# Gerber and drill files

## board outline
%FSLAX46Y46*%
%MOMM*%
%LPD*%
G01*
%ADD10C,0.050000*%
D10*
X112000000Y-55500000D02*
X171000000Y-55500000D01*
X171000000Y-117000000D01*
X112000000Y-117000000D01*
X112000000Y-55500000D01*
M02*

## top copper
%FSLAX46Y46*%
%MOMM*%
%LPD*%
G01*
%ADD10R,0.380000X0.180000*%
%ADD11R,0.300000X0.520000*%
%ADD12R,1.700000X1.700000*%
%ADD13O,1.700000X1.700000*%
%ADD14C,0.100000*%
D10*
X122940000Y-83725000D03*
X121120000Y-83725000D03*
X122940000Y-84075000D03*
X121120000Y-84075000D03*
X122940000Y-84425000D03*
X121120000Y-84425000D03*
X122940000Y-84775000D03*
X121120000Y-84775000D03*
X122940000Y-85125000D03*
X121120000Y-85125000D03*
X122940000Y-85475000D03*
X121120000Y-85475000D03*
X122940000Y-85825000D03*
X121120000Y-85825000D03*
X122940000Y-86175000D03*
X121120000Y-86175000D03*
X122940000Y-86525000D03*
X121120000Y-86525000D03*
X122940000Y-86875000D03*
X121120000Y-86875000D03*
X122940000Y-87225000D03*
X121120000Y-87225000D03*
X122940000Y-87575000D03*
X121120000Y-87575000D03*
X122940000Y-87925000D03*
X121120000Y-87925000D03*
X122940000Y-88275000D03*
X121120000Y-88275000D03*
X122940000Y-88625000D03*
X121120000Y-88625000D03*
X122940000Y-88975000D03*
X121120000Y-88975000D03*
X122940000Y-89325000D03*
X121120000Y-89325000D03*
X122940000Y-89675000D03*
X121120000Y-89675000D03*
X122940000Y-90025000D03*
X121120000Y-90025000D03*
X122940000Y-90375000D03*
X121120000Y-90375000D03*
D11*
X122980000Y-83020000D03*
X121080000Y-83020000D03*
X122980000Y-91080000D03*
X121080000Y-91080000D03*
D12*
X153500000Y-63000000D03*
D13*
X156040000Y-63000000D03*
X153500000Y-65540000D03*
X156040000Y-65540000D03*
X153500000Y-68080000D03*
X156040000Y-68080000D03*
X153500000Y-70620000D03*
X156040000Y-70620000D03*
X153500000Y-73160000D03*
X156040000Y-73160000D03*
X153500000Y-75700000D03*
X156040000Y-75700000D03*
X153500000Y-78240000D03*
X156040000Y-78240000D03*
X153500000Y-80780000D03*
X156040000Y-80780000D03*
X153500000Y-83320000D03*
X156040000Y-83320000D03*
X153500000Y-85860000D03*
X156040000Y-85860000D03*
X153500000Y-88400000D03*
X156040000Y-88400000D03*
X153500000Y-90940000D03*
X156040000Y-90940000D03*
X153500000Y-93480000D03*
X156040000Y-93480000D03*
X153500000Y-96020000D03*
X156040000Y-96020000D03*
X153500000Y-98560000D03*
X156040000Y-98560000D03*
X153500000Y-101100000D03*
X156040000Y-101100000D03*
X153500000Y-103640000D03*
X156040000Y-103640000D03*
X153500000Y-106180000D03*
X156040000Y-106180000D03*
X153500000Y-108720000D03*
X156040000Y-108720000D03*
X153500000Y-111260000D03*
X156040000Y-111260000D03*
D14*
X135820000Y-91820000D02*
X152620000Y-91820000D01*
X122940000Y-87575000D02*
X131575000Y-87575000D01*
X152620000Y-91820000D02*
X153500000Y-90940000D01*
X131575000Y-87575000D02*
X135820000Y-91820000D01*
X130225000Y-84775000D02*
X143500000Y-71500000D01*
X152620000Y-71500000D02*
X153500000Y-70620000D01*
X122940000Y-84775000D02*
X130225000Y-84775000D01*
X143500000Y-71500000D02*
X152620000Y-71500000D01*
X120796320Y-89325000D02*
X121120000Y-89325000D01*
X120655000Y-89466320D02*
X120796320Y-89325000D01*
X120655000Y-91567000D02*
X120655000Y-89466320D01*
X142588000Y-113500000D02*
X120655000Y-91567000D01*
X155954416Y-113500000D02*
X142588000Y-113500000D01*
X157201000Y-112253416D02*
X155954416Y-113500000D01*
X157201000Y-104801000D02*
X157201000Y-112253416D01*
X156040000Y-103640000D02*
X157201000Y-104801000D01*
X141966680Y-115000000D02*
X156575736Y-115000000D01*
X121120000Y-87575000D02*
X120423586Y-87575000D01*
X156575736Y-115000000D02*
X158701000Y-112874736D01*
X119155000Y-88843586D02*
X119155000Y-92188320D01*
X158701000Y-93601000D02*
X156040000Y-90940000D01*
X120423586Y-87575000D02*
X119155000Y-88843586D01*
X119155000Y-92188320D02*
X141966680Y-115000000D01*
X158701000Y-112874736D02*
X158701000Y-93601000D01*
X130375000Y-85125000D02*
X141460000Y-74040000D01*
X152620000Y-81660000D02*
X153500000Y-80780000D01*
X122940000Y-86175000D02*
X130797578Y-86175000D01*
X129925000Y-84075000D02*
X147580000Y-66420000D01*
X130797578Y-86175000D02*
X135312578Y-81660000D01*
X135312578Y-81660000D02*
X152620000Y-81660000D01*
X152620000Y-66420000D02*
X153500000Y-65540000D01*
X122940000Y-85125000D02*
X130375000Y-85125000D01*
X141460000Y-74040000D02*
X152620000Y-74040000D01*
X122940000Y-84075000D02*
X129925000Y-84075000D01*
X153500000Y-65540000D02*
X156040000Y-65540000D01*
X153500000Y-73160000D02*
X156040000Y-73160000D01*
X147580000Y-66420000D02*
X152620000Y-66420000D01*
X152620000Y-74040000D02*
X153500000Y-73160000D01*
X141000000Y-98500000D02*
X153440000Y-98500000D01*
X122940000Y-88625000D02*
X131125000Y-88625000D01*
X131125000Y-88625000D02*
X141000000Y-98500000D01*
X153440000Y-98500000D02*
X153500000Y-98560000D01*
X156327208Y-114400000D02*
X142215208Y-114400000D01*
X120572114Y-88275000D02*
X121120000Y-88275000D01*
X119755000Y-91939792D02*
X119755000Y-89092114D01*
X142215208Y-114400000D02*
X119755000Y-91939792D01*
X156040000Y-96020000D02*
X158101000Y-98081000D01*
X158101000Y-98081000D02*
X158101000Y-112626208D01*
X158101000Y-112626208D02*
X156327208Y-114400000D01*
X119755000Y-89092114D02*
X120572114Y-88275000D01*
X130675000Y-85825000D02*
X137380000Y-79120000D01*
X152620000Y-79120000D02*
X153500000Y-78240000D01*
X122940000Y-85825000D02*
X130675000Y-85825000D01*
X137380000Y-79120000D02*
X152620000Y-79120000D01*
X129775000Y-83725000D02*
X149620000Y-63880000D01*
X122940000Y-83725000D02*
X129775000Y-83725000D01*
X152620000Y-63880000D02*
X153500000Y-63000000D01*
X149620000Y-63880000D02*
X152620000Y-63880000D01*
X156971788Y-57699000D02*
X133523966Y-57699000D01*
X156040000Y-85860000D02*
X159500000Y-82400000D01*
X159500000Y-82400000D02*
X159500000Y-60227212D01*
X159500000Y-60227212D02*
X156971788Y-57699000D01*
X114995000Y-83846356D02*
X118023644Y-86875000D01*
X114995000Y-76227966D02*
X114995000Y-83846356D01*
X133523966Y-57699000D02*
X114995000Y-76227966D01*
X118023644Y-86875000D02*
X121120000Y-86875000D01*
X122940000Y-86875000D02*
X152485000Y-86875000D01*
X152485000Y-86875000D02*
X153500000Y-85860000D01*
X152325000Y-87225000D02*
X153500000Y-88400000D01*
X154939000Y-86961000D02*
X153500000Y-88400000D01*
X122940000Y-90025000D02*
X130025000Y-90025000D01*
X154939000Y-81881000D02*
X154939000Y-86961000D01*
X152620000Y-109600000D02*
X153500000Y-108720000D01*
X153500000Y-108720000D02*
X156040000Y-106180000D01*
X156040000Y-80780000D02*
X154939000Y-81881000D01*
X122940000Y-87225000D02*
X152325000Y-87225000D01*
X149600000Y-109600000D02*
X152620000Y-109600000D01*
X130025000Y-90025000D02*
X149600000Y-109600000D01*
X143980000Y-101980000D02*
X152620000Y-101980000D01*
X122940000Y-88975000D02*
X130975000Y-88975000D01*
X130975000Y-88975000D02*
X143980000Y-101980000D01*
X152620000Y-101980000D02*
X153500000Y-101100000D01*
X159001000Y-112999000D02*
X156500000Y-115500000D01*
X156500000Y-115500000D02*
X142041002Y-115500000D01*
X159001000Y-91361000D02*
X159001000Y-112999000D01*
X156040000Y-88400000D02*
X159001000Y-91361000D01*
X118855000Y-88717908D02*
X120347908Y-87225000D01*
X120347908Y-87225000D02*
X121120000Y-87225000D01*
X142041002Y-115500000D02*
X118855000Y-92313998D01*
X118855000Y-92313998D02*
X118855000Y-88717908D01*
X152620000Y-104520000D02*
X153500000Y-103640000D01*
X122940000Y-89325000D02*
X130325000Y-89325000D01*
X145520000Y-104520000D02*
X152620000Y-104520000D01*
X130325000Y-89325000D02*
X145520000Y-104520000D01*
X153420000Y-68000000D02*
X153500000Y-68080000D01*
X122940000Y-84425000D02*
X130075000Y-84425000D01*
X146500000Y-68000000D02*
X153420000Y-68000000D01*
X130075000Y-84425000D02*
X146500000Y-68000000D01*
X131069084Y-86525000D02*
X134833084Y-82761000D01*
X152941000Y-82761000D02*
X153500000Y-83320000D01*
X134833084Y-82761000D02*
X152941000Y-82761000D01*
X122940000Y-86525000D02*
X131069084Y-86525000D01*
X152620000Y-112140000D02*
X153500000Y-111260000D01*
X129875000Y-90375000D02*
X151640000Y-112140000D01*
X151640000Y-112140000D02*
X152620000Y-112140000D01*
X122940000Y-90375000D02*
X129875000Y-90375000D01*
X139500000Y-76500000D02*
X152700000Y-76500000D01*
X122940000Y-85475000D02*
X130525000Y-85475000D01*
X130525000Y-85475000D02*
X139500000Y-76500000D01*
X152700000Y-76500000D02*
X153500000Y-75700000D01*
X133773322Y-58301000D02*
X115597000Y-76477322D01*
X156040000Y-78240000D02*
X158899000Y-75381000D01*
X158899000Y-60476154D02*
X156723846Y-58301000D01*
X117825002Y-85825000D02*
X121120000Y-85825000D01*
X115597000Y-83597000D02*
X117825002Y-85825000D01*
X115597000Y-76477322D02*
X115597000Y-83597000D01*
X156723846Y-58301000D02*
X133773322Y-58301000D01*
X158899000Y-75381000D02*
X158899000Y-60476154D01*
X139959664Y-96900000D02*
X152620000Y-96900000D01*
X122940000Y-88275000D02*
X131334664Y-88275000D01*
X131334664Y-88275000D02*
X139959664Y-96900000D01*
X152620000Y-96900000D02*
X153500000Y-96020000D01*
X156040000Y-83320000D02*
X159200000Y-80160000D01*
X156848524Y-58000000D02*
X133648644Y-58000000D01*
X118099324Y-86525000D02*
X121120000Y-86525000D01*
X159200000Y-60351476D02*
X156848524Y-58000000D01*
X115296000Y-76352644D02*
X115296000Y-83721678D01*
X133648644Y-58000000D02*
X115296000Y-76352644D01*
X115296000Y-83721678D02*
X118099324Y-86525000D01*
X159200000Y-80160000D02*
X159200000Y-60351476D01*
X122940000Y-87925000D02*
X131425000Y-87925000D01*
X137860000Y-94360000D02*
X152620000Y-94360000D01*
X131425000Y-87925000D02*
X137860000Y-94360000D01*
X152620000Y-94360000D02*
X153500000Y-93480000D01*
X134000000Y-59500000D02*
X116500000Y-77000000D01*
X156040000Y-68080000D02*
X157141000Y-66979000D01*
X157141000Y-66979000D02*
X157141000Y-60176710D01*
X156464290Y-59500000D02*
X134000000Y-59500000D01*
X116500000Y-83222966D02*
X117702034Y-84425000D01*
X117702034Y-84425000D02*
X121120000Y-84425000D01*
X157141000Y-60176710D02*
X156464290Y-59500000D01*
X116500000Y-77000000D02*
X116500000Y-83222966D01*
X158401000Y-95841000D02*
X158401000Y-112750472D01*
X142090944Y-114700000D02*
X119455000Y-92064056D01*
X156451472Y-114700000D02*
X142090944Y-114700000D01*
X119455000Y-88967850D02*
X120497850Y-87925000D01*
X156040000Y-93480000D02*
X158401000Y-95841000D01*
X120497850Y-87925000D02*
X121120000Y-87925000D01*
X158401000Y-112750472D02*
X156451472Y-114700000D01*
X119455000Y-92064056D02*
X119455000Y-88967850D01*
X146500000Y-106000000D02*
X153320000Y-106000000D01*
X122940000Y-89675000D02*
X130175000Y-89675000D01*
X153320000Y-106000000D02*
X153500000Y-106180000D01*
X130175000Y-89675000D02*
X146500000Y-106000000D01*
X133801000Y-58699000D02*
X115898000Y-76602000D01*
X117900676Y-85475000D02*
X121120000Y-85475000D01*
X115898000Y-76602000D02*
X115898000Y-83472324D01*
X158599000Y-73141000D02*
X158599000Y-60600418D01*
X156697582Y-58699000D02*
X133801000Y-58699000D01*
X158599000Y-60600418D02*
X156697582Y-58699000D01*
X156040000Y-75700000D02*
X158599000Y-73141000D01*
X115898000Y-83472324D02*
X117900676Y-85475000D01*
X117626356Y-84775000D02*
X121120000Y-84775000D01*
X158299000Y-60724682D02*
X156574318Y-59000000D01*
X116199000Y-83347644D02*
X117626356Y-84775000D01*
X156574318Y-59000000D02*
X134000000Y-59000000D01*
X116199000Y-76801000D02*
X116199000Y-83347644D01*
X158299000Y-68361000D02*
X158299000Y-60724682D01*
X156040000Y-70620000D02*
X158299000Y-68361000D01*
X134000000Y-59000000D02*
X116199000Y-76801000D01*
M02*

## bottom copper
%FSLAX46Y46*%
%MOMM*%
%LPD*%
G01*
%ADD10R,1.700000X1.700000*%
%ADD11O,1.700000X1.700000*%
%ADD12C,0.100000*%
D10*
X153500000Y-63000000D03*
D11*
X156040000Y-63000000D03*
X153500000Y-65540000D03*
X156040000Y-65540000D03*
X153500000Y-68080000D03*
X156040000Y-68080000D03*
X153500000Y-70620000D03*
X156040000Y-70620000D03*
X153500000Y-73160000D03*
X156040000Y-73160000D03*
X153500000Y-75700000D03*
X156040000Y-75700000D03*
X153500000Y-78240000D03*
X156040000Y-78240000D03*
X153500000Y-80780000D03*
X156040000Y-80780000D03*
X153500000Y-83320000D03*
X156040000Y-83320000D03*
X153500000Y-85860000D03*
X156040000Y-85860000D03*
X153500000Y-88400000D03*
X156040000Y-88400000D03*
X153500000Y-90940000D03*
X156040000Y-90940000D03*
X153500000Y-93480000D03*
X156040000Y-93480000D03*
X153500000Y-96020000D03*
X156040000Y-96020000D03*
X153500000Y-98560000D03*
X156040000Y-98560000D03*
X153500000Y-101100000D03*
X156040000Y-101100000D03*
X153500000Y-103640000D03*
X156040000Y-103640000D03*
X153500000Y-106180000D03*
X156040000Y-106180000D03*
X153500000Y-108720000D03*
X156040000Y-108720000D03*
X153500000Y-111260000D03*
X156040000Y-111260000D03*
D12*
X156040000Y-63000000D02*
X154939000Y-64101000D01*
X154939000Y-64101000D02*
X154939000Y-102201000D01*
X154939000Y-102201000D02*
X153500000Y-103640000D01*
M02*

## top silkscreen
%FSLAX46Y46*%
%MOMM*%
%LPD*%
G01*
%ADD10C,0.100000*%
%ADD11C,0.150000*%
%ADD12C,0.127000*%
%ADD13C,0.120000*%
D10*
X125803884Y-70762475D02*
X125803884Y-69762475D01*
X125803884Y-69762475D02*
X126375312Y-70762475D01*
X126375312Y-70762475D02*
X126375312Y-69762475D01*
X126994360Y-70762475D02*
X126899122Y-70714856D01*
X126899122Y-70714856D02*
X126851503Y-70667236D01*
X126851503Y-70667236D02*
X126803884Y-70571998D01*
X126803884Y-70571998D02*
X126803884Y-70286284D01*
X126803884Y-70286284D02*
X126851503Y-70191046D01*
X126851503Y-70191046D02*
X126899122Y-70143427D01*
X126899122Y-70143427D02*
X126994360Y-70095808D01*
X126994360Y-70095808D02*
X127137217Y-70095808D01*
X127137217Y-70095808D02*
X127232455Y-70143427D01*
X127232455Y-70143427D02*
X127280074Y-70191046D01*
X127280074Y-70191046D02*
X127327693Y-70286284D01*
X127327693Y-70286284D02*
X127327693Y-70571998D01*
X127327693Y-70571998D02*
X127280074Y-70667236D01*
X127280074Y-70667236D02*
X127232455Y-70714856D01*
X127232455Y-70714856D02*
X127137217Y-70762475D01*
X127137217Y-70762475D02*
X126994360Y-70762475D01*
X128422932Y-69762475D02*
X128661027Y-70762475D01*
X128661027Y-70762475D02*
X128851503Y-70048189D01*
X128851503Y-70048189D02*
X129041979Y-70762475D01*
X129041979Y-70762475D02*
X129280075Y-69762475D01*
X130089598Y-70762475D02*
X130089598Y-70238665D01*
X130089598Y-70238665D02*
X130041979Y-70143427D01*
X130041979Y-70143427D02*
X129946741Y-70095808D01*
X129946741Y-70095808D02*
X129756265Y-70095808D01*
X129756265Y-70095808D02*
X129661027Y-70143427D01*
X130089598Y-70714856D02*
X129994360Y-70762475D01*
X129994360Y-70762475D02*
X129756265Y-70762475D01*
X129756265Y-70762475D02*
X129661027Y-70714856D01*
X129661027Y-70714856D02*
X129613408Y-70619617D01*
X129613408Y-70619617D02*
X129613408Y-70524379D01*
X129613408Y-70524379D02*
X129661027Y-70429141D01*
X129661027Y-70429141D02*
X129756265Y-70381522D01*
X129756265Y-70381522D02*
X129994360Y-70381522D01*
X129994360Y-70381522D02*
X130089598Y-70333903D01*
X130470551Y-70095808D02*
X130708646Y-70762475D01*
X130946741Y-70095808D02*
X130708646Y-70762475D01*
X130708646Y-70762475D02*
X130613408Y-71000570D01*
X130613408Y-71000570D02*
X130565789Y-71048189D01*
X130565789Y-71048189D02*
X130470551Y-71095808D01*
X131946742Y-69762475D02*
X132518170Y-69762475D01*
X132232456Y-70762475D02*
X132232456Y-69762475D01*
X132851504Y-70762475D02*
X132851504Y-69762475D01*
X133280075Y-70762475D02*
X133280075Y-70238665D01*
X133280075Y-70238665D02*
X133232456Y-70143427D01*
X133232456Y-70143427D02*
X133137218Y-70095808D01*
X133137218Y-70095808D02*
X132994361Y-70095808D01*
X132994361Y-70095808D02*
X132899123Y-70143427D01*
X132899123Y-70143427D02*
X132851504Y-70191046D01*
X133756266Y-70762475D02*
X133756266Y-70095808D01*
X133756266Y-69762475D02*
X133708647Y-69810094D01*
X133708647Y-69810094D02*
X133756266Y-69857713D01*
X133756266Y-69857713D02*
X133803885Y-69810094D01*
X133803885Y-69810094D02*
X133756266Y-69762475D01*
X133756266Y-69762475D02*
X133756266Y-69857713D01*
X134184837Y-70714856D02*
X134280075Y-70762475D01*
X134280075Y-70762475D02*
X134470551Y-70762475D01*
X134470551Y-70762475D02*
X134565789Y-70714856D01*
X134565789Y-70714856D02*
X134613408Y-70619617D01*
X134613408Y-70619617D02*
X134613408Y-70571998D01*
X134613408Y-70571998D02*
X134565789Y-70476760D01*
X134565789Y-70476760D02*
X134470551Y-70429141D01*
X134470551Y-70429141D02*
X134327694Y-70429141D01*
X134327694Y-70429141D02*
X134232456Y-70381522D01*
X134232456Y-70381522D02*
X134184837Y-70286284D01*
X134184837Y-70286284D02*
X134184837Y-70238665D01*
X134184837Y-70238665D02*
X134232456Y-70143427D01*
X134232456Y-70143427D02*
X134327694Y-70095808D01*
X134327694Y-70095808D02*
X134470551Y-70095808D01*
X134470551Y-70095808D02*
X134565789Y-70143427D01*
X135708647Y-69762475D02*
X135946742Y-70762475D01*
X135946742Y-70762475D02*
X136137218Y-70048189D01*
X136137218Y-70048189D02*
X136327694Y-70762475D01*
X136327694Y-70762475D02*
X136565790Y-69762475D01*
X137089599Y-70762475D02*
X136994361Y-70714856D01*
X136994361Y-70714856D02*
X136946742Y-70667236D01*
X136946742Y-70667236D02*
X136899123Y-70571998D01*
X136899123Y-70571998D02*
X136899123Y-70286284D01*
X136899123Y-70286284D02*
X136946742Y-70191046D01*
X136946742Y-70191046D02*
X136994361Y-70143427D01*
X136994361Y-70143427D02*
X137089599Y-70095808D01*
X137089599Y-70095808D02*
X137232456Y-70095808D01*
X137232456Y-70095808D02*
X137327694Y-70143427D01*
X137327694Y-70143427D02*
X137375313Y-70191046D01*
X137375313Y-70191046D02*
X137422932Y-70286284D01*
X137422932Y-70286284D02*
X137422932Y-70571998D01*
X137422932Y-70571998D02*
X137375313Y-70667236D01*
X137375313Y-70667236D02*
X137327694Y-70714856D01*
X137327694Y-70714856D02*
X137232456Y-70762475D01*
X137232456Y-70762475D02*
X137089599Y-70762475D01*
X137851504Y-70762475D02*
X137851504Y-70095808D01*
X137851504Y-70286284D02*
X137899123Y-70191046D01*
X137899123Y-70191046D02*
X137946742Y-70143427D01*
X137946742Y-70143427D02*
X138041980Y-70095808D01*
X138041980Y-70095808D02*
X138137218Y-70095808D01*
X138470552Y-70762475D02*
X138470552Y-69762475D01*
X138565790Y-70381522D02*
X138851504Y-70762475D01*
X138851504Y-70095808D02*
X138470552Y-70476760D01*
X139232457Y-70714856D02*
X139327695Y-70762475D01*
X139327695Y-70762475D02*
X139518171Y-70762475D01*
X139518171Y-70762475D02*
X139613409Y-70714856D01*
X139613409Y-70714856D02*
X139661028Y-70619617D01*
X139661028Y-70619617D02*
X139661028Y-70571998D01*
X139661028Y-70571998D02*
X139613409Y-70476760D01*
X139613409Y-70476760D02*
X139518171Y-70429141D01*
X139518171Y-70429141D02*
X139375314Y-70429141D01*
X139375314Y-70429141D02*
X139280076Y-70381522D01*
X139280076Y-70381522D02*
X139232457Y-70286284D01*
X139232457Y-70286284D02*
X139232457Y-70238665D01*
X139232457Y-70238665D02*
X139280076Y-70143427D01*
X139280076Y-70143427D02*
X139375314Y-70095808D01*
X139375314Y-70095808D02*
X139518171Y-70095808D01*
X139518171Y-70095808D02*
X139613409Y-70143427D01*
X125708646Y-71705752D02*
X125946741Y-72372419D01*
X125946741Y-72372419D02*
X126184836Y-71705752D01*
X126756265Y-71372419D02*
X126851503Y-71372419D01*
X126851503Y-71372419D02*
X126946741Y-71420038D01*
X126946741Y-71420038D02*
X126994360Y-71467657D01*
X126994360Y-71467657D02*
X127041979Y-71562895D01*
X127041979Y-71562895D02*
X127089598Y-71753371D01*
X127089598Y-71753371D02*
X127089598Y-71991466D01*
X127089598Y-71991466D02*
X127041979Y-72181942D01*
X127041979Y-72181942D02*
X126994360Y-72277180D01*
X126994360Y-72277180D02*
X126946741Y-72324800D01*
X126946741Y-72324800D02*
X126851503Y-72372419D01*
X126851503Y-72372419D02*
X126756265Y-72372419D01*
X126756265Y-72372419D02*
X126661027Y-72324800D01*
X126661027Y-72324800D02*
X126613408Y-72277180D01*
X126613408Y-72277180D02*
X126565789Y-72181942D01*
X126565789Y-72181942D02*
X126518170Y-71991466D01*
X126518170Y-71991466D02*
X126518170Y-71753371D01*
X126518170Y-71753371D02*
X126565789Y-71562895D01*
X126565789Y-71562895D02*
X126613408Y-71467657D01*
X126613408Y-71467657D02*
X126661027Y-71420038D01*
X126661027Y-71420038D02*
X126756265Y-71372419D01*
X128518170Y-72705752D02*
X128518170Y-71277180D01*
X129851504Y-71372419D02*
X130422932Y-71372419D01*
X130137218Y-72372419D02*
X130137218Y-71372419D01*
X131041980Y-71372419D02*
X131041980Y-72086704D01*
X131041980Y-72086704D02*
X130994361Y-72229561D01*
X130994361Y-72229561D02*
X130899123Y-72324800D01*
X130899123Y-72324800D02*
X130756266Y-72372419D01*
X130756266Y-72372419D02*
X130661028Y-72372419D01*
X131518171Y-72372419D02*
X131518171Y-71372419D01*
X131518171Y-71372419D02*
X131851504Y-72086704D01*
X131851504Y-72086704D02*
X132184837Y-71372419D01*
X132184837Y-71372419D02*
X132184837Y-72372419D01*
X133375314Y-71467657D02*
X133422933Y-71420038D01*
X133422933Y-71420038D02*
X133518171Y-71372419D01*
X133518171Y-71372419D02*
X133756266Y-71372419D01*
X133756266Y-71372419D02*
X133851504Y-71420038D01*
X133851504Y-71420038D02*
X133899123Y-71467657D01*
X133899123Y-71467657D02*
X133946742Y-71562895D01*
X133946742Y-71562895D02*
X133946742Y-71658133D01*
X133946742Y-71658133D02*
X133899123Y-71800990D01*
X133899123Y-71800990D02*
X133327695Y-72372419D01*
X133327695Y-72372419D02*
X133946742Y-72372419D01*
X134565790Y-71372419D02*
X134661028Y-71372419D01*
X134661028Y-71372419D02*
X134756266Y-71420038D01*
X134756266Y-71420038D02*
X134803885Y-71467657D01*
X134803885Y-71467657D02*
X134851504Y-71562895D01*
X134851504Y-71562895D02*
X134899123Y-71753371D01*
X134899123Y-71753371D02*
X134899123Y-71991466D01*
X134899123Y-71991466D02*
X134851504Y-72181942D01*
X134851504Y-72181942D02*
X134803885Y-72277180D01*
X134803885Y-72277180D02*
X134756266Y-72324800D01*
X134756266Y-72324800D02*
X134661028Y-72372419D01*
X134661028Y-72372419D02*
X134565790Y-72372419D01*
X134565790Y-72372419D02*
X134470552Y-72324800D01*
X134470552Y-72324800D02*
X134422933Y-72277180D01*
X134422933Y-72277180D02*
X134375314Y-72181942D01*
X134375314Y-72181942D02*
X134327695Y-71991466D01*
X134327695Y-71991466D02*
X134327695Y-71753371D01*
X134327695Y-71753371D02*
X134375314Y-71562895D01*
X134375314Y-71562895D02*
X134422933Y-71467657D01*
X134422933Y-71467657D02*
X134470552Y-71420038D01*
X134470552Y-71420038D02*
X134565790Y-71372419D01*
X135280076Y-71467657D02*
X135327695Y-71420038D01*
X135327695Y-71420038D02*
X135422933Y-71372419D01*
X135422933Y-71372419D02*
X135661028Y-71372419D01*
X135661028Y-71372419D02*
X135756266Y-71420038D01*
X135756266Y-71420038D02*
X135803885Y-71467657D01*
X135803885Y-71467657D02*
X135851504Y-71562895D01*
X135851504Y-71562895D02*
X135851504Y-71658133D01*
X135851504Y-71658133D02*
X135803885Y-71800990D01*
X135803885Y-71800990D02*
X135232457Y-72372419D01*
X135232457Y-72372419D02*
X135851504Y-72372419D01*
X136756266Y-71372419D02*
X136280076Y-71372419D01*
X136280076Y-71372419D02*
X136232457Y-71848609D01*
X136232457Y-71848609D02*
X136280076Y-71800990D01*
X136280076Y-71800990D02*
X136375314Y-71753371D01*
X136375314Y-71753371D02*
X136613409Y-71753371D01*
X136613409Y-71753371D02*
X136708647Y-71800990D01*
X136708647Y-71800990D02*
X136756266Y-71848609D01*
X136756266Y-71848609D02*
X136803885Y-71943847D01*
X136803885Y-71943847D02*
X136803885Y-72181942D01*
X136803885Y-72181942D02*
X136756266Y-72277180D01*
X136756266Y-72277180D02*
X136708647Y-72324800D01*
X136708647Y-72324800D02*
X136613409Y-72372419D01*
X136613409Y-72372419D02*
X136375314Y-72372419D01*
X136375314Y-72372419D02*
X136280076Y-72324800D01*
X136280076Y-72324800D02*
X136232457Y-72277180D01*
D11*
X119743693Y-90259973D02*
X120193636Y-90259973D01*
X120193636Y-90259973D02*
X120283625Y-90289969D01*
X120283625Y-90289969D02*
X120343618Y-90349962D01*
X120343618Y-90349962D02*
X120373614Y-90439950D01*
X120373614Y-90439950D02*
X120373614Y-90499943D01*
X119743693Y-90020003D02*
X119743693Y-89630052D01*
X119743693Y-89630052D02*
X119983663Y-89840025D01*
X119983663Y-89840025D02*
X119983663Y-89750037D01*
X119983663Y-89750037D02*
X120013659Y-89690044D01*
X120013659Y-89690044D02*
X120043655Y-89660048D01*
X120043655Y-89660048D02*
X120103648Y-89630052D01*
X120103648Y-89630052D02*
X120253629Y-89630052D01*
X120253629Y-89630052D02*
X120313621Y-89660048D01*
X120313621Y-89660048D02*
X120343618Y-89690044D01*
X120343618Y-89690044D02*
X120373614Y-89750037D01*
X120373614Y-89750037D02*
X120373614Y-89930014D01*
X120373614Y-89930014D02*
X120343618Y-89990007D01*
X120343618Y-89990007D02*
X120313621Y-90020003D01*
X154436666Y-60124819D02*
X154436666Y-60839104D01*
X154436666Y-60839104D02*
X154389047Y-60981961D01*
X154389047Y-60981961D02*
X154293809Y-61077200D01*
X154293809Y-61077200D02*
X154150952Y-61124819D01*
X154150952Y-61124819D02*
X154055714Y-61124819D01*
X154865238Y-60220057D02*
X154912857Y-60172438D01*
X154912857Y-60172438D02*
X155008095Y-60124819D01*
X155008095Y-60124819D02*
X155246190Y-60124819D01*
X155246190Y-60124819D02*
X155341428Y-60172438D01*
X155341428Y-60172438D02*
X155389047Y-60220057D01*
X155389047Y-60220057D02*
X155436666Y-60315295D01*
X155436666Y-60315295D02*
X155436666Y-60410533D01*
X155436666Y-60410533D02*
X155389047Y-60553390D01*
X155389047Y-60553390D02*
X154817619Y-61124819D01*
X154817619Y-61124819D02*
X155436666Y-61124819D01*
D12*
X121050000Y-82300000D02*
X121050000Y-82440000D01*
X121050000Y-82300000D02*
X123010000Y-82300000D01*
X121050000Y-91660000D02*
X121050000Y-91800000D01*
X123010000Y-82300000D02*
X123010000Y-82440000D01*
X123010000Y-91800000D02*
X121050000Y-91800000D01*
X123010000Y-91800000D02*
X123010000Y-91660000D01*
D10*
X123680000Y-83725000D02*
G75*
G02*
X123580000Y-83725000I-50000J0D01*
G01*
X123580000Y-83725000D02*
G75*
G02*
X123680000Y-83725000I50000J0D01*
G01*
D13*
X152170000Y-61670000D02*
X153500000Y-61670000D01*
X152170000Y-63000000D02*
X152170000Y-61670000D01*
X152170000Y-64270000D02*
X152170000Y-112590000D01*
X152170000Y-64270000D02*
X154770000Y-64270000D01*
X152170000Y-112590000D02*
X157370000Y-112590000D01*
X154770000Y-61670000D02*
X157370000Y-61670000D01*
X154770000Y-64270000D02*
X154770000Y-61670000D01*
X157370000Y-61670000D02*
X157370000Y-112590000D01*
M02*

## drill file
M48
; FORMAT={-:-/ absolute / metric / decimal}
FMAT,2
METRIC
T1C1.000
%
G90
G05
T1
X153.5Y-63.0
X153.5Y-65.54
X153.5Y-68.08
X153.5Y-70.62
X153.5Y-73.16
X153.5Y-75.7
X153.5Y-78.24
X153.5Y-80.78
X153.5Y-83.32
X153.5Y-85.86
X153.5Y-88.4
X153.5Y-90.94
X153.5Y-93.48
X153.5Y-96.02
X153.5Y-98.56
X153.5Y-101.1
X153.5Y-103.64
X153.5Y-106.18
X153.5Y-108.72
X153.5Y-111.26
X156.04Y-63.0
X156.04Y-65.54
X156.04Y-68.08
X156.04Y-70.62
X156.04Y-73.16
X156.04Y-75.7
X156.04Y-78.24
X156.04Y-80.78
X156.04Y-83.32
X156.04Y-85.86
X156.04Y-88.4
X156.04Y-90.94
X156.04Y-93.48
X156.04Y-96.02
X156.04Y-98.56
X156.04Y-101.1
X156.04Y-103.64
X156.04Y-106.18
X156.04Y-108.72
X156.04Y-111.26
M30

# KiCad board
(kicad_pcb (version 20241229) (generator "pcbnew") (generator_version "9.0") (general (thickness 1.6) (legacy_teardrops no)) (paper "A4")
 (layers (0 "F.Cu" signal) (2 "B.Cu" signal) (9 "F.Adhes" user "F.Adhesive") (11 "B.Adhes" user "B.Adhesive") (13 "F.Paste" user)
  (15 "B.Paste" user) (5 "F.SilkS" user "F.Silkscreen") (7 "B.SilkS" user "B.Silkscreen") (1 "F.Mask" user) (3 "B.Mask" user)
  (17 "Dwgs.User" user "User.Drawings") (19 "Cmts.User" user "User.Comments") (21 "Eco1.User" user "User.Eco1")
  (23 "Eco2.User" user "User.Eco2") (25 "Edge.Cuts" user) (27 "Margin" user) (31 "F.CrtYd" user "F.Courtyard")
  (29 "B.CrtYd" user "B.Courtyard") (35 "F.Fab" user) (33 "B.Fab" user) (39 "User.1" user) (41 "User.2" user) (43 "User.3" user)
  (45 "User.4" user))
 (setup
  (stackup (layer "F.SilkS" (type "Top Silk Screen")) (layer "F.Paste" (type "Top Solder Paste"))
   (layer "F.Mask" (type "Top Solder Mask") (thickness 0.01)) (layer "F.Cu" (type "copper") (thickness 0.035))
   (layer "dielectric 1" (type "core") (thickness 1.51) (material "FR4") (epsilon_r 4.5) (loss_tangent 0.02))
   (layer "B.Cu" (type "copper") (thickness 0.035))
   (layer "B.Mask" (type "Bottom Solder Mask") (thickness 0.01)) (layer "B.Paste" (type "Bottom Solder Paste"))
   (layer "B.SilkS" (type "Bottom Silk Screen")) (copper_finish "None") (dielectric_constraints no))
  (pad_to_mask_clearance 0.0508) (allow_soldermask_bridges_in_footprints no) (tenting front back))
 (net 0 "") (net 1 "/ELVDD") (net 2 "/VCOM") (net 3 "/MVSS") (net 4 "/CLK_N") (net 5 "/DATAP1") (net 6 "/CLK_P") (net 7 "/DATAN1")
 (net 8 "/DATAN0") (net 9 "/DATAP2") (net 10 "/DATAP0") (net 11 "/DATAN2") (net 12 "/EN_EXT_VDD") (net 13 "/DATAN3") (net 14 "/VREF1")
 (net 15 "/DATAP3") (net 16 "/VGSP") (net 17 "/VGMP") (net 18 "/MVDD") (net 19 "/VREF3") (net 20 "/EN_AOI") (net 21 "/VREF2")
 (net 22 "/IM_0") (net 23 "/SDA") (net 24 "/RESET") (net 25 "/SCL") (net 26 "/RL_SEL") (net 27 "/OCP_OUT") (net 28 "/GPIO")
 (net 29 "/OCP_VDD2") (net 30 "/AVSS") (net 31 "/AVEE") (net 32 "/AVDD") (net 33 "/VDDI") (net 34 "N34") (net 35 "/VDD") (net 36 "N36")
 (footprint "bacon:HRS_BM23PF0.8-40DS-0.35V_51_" (layer "F.Cu") (at 122.03 87.05 90)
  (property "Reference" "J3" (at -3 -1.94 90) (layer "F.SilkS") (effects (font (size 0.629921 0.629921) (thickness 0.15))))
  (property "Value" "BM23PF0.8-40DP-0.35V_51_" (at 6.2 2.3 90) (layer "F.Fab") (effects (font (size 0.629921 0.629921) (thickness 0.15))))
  (fp_line (start 4.75 -0.98) (end 4.61 -0.98) (stroke (width 0.127) (type solid)) (layer "F.SilkS"))
  (fp_line (start 4.75 -0.98) (end 4.75 0.98) (stroke (width 0.127) (type solid)) (layer "F.SilkS"))
  (fp_line (start -4.61 -0.98) (end -4.75 -0.98) (stroke (width 0.127) (type solid)) (layer "F.SilkS"))
  (fp_line (start 4.75 0.98) (end 4.61 0.98) (stroke (width 0.127) (type solid)) (layer "F.SilkS"))
  (fp_line (start -4.75 0.98) (end -4.75 -0.98) (stroke (width 0.127) (type solid)) (layer "F.SilkS"))
  (fp_line (start -4.75 0.98) (end -4.61 0.98) (stroke (width 0.127) (type solid)) (layer "F.SilkS"))
  (fp_circle (center 3.325 1.6) (end 3.375 1.6) (stroke (width 0.1) (type solid)) (fill no) (layer "F.SilkS"))
  (pad "1" smd rect (at 3.325 0.91 90) (size 0.18 0.38) (layers "F.Cu" "F.Paste") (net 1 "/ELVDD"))
  (pad "2" smd rect (at 3.325 -0.91 90) (size 0.18 0.38) (layers "F.Cu" "F.Paste") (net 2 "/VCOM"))
  (pad "3" smd rect (at 2.975 0.91 90) (size 0.18 0.38) (layers "F.Cu" "F.Paste") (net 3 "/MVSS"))
  (pad "4" smd rect (at 2.975 -0.91 90) (size 0.18 0.38) (layers "F.Cu" "F.Paste") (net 3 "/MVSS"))
  (pad "5" smd rect (at 2.625 0.91 90) (size 0.18 0.38) (layers "F.Cu" "F.Paste") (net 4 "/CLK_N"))
  (pad "6" smd rect (at 2.625 -0.91 90) (size 0.18 0.38) (layers "F.Cu" "F.Paste") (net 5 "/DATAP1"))
  (pad "7" smd rect (at 2.275 0.91 90) (size 0.18 0.38) (layers "F.Cu" "F.Paste") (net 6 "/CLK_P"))
  (pad "8" smd rect (at 2.275 -0.91 90) (size 0.18 0.38) (layers "F.Cu" "F.Paste") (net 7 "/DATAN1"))
  (pad "9" smd rect (at 1.925 0.91 90) (size 0.18 0.38) (layers "F.Cu" "F.Paste") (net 3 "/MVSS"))
  (pad "10" smd rect (at 1.925 -0.91 90) (size 0.18 0.38) (layers "F.Cu" "F.Paste") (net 3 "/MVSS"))
  (pad "11" smd rect (at 1.575 0.91 90) (size 0.18 0.38) (layers "F.Cu" "F.Paste") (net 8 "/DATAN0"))
  (pad "12" smd rect (at 1.575 -0.91 90) (size 0.18 0.38) (layers "F.Cu" "F.Paste") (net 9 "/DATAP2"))
  (pad "13" smd rect (at 1.225 0.91 90) (size 0.18 0.38) (layers "F.Cu" "F.Paste") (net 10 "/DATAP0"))
  (pad "14" smd rect (at 1.225 -0.91 90) (size 0.18 0.38) (layers "F.Cu" "F.Paste") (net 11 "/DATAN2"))
  (pad "15" smd rect (at 0.875 0.91 90) (size 0.18 0.38) (layers "F.Cu" "F.Paste") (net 3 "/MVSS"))
  (pad "16" smd rect (at 0.875 -0.91 90) (size 0.18 0.38) (layers "F.Cu" "F.Paste") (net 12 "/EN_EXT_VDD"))
  (pad "17" smd rect (at 0.525 0.91 90) (size 0.18 0.38) (layers "F.Cu" "F.Paste") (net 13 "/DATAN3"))
  (pad "18" smd rect (at 0.525 -0.91 90) (size 0.18 0.38) (layers "F.Cu" "F.Paste") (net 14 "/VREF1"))
  (pad "19" smd rect (at 0.175 0.91 90) (size 0.18 0.38) (layers "F.Cu" "F.Paste") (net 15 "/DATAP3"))
  (pad "20" smd rect (at 0.175 -0.91 90) (size 0.18 0.38) (layers "F.Cu" "F.Paste") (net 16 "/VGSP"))
  (pad "21" smd rect (at -0.175 0.91 90) (size 0.18 0.38) (layers "F.Cu" "F.Paste") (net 12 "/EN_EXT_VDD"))
  (pad "22" smd rect (at -0.175 -0.91 90) (size 0.18 0.38) (layers "F.Cu" "F.Paste") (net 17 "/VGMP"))
  (pad "23" smd rect (at -0.525 0.91 90) (size 0.18 0.38) (layers "F.Cu" "F.Paste") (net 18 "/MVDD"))
  (pad "24" smd rect (at -0.525 -0.91 90) (size 0.18 0.38) (layers "F.Cu" "F.Paste") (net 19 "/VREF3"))
  (pad "25" smd rect (at -0.875 0.91 90) (size 0.18 0.38) (layers "F.Cu" "F.Paste") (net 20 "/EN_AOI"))
  (pad "26" smd rect (at -0.875 -0.91 90) (size 0.18 0.38) (layers "F.Cu" "F.Paste") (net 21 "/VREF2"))
  (pad "27" smd rect (at -1.225 0.91 90) (size 0.18 0.38) (layers "F.Cu" "F.Paste") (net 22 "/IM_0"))
  (pad "28" smd rect (at -1.225 -0.91 90) (size 0.18 0.38) (layers "F.Cu" "F.Paste") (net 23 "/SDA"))
  (pad "29" smd rect (at -1.575 0.91 90) (size 0.18 0.38) (layers "F.Cu" "F.Paste") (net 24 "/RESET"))
  (pad "30" smd rect (at -1.575 -0.91 90) (size 0.18 0.38) (layers "F.Cu" "F.Paste") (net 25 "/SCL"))
  (pad "31" smd rect (at -1.925 0.91 90) (size 0.18 0.38) (layers "F.Cu" "F.Paste") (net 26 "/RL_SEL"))
  (pad "32" smd rect (at -1.925 -0.91 90) (size 0.18 0.38) (layers "F.Cu" "F.Paste") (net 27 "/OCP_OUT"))
  (pad "33" smd rect (at -2.275 0.91 90) (size 0.18 0.38) (layers "F.Cu" "F.Paste") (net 2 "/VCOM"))
  (pad "34" smd rect (at -2.275 -0.91 90) (size 0.18 0.38) (layers "F.Cu" "F.Paste") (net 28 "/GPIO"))
  (pad "35" smd rect (at -2.625 0.91 90) (size 0.18 0.38) (layers "F.Cu" "F.Paste") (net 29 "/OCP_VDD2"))
  (pad "36" smd rect (at -2.625 -0.91 90) (size 0.18 0.38) (layers "F.Cu" "F.Paste") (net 12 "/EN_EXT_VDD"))
  (pad "37" smd rect (at -2.975 0.91 90) (size 0.18 0.38) (layers "F.Cu" "F.Paste") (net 12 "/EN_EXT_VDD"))
  (pad "38" smd rect (at -2.975 -0.91 90) (size 0.18 0.38) (layers "F.Cu" "F.Paste") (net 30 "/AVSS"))
  (pad "39" smd rect (at -3.325 0.91 90) (size 0.18 0.38) (layers "F.Cu" "F.Paste") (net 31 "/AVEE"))
  (pad "40" smd rect (at -3.325 -0.91 90) (size 0.18 0.38) (layers "F.Cu" "F.Paste") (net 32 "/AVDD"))
  (pad "P1_1" smd rect (at 4.03 0.95 90) (size 0.52 0.3) (layers "F.Cu" "F.Mask" "F.Paste") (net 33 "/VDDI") (solder_mask_margin 0.102))
  (pad "P1_2" smd rect (at 4.03 -0.95 90) (size 0.52 0.3) (layers "F.Cu" "F.Mask" "F.Paste") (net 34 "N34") (solder_mask_margin 0.102))
  (pad "P2_1" smd rect (at -4.03 0.95 90) (size 0.52 0.3) (layers "F.Cu" "F.Mask" "F.Paste") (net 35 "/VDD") (solder_mask_margin 0.102))
  (pad "P2_2" smd rect (at -4.03 -0.95 90) (size 0.52 0.3) (layers "F.Cu" "F.Mask" "F.Paste") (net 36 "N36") (solder_mask_margin 0.102)))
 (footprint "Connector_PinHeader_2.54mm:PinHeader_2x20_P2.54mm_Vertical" (layer "F.Cu") (at 153.5 63)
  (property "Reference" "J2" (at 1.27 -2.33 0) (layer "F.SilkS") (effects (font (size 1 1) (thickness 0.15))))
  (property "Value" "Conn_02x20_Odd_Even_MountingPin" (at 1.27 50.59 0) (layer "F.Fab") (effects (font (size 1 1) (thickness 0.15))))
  (fp_line (start -1.33 -1.33) (end 0 -1.33) (stroke (width 0.12) (type solid)) (layer "F.SilkS"))
  (fp_line (start -1.33 0) (end -1.33 -1.33) (stroke (width 0.12) (type solid)) (layer "F.SilkS"))
  (fp_line (start -1.33 1.27) (end -1.33 49.59) (stroke (width 0.12) (type solid)) (layer "F.SilkS"))
  (fp_line (start -1.33 1.27) (end 1.27 1.27) (stroke (width 0.12) (type solid)) (layer "F.SilkS"))
  (fp_line (start -1.33 49.59) (end 3.87 49.59) (stroke (width 0.12) (type solid)) (layer "F.SilkS"))
  (fp_line (start 1.27 -1.33) (end 3.87 -1.33) (stroke (width 0.12) (type solid)) (layer "F.SilkS"))
  (fp_line (start 1.27 1.27) (end 1.27 -1.33) (stroke (width 0.12) (type solid)) (layer "F.SilkS"))
  (fp_line (start 3.87 -1.33) (end 3.87 49.59) (stroke (width 0.12) (type solid)) (layer "F.SilkS"))
  (pad "1" thru_hole rect (at 0 0) (size 1.7 1.7) (drill 1) (layers "*.Cu" "*.Mask") (remove_unused_layers no) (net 1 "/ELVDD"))
  (pad "2" thru_hole oval (at 2.54 0) (size 1.7 1.7) (drill 1) (layers "*.Cu" "*.Mask") (remove_unused_layers no) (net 2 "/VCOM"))
  (pad "3" thru_hole oval (at 0 2.54) (size 1.7 1.7) (drill 1) (layers "*.Cu" "*.Mask") (remove_unused_layers no) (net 3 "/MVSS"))
  (pad "4" thru_hole oval (at 2.54 2.54) (size 1.7 1.7) (drill 1) (layers "*.Cu" "*.Mask") (remove_unused_layers no) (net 3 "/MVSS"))
  (pad "5" thru_hole oval (at 0 5.08) (size 1.7 1.7) (drill 1) (layers "*.Cu" "*.Mask") (remove_unused_layers no) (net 4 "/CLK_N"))
  (pad "6" thru_hole oval (at 2.54 5.08) (size 1.7 1.7) (drill 1) (layers "*.Cu" "*.Mask") (remove_unused_layers no) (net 5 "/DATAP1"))
  (pad "7" thru_hole oval (at 0 7.62) (size 1.7 1.7) (drill 1) (layers "*.Cu" "*.Mask") (remove_unused_layers no) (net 6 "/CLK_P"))
  (pad "8" thru_hole oval (at 2.54 7.62) (size 1.7 1.7) (drill 1) (layers "*.Cu" "*.Mask") (remove_unused_layers no) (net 7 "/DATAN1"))
  (pad "9" thru_hole oval (at 0 10.16) (size 1.7 1.7) (drill 1) (layers "*.Cu" "*.Mask") (remove_unused_layers no) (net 3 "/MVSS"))
  (pad "10" thru_hole oval (at 2.54 10.16) (size 1.7 1.7) (drill 1) (layers "*.Cu" "*.Mask") (remove_unused_layers no) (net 3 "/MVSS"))
  (pad "11" thru_hole oval (at 0 12.7) (size 1.7 1.7) (drill 1) (layers "*.Cu" "*.Mask") (remove_unused_layers no) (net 8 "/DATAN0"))
  (pad "12" thru_hole oval (at 2.54 12.7) (size 1.7 1.7) (drill 1) (layers "*.Cu" "*.Mask") (remove_unused_layers no) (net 9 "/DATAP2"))
  (pad "13" thru_hole oval (at 0 15.24) (size 1.7 1.7) (drill 1) (layers "*.Cu" "*.Mask") (remove_unused_layers no) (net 10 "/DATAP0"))
  (pad "14" thru_hole oval (at 2.54 15.24) (size 1.7 1.7) (drill 1) (layers "*.Cu" "*.Mask") (remove_unused_layers no) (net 11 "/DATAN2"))
  (pad "15" thru_hole oval (at 0 17.78) (size 1.7 1.7) (drill 1) (layers "*.Cu" "*.Mask") (remove_unused_layers no) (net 3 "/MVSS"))
  (pad "16" thru_hole oval (at 2.54 17.78) (size 1.7 1.7) (drill 1) (layers "*.Cu" "*.Mask") (remove_unused_layers no)
   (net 12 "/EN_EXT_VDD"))
  (pad "17" thru_hole oval (at 0 20.32) (size 1.7 1.7) (drill 1) (layers "*.Cu" "*.Mask") (remove_unused_layers no) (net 13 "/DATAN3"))
  (pad "18" thru_hole oval (at 2.54 20.32) (size 1.7 1.7) (drill 1) (layers "*.Cu" "*.Mask") (remove_unused_layers no) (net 14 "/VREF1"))
  (pad "19" thru_hole oval (at 0 22.86) (size 1.7 1.7) (drill 1) (layers "*.Cu" "*.Mask") (remove_unused_layers no) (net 15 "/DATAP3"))
  (pad "20" thru_hole oval (at 2.54 22.86) (size 1.7 1.7) (drill 1) (layers "*.Cu" "*.Mask") (remove_unused_layers no) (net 16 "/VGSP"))
  (pad "21" thru_hole oval (at 0 25.4) (size 1.7 1.7) (drill 1) (layers "*.Cu" "*.Mask") (remove_unused_layers no) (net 12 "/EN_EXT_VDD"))
  (pad "22" thru_hole oval (at 2.54 25.4) (size 1.7 1.7) (drill 1) (layers "*.Cu" "*.Mask") (remove_unused_layers no) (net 17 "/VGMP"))
  (pad "23" thru_hole oval (at 0 27.94) (size 1.7 1.7) (drill 1) (layers "*.Cu" "*.Mask") (remove_unused_layers no) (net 18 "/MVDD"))
  (pad "24" thru_hole oval (at 2.54 27.94) (size 1.7 1.7) (drill 1) (layers "*.Cu" "*.Mask") (remove_unused_layers no) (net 19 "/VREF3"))
  (pad "25" thru_hole oval (at 0 30.48) (size 1.7 1.7) (drill 1) (layers "*.Cu" "*.Mask") (remove_unused_layers no) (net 20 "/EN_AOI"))
  (pad "26" thru_hole oval (at 2.54 30.48) (size 1.7 1.7) (drill 1) (layers "*.Cu" "*.Mask") (remove_unused_layers no) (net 21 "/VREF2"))
  (pad "27" thru_hole oval (at 0 33.02) (size 1.7 1.7) (drill 1) (layers "*.Cu" "*.Mask") (remove_unused_layers no) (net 22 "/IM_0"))
  (pad "28" thru_hole oval (at 2.54 33.02) (size 1.7 1.7) (drill 1) (layers "*.Cu" "*.Mask") (remove_unused_layers no) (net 23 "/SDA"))
  (pad "29" thru_hole oval (at 0 35.56) (size 1.7 1.7) (drill 1) (layers "*.Cu" "*.Mask") (remove_unused_layers no) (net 24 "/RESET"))
  (pad "30" thru_hole oval (at 2.54 35.56) (size 1.7 1.7) (drill 1) (layers "*.Cu" "*.Mask") (remove_unused_layers no) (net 25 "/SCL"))
  (pad "31" thru_hole oval (at 0 38.1) (size 1.7 1.7) (drill 1) (layers "*.Cu" "*.Mask") (remove_unused_layers no) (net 26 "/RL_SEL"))
  (pad "32" thru_hole oval (at 2.54 38.1) (size 1.7 1.7) (drill 1) (layers "*.Cu" "*.Mask") (remove_unused_layers no) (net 27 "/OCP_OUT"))
  (pad "33" thru_hole oval (at 0 40.64) (size 1.7 1.7) (drill 1) (layers "*.Cu" "*.Mask") (remove_unused_layers no) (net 2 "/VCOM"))
  (pad "34" thru_hole oval (at 2.54 40.64) (size 1.7 1.7) (drill 1) (layers "*.Cu" "*.Mask") (remove_unused_layers no) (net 28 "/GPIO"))
  (pad "35" thru_hole oval (at 0 43.18) (size 1.7 1.7) (drill 1) (layers "*.Cu" "*.Mask") (remove_unused_layers no) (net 29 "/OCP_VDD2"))
  (pad "36" thru_hole oval (at 2.54 43.18) (size 1.7 1.7) (drill 1) (layers "*.Cu" "*.Mask") (remove_unused_layers no)
   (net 12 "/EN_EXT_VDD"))
  (pad "37" thru_hole oval (at 0 45.72) (size 1.7 1.7) (drill 1) (layers "*.Cu" "*.Mask") (remove_unused_layers no) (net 12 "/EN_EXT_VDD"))
  (pad "38" thru_hole oval (at 2.54 45.72) (size 1.7 1.7) (drill 1) (layers "*.Cu" "*.Mask") (remove_unused_layers no) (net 30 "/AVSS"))
  (pad "39" thru_hole oval (at 0 48.26) (size 1.7 1.7) (drill 1) (layers "*.Cu" "*.Mask") (remove_unused_layers no) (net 31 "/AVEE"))
  (pad "40" thru_hole oval (at 2.54 48.26) (size 1.7 1.7) (drill 1) (layers "*.Cu" "*.Mask") (remove_unused_layers no) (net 32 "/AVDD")))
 (gr_rect (start 112 55.5) (end 171 117) (stroke (width 0.05) (type default)) (fill no) (layer "Edge.Cuts"))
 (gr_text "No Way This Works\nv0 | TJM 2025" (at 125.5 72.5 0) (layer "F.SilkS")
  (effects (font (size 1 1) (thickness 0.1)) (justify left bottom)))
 (segment (start 135.82 91.82) (end 152.62 91.82) (width 0.1) (layer "F.Cu") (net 18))
 (segment (start 122.94 87.575) (end 131.575 87.575) (width 0.1) (layer "F.Cu") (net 18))
 (segment (start 152.62 91.82) (end 153.5 90.94) (width 0.1) (layer "F.Cu") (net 18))
 (segment (start 131.575 87.575) (end 135.82 91.82) (width 0.1) (layer "F.Cu") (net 18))
 (segment (start 130.225 84.775) (end 143.5 71.5) (width 0.1) (layer "F.Cu") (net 6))
 (segment (start 152.62 71.5) (end 153.5 70.62) (width 0.1) (layer "F.Cu") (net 6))
 (segment (start 122.94 84.775) (end 130.225 84.775) (width 0.1) (layer "F.Cu") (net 6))
 (segment (start 143.5 71.5) (end 152.62 71.5) (width 0.1) (layer "F.Cu") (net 6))
 (segment (start 120.79632 89.325) (end 121.12 89.325) (width 0.1) (layer "F.Cu") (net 28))
 (segment (start 120.655 89.46632) (end 120.79632 89.325) (width 0.1) (layer "F.Cu") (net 28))
 (segment (start 120.655 91.567) (end 120.655 89.46632) (width 0.1) (layer "F.Cu") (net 28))
 (segment (start 142.588 113.5) (end 120.655 91.567) (width 0.1) (layer "F.Cu") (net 28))
 (segment (start 155.954416 113.5) (end 142.588 113.5) (width 0.1) (layer "F.Cu") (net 28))
 (segment (start 157.201 112.253416) (end 155.954416 113.5) (width 0.1) (layer "F.Cu") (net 28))
 (segment (start 157.201 104.801) (end 157.201 112.253416) (width 0.1) (layer "F.Cu") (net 28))
 (segment (start 156.04 103.64) (end 157.201 104.801) (width 0.1) (layer "F.Cu") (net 28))
 (segment (start 141.96668 115) (end 156.575736 115) (width 0.1) (layer "F.Cu") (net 19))
 (segment (start 121.12 87.575) (end 120.423586 87.575) (width 0.1) (layer "F.Cu") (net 19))
 (segment (start 156.575736 115) (end 158.701 112.874736) (width 0.1) (layer "F.Cu") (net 19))
 (segment (start 119.155 88.843586) (end 119.155 92.18832) (width 0.1) (layer "F.Cu") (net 19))
 (segment (start 158.701 93.601) (end 156.04 90.94) (width 0.1) (layer "F.Cu") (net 19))
 (segment (start 120.423586 87.575) (end 119.155 88.843586) (width 0.1) (layer "F.Cu") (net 19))
 (segment (start 119.155 92.18832) (end 141.96668 115) (width 0.1) (layer "F.Cu") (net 19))
 (segment (start 158.701 112.874736) (end 158.701 93.601) (width 0.1) (layer "F.Cu") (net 19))
 (segment (start 130.375 85.125) (end 141.46 74.04) (width 0.1) (layer "F.Cu") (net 3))
 (segment (start 152.62 81.66) (end 153.5 80.78) (width 0.1) (layer "F.Cu") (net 3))
 (segment (start 122.94 86.175) (end 130.797578 86.175) (width 0.1) (layer "F.Cu") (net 3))
 (segment (start 129.925 84.075) (end 147.58 66.42) (width 0.1) (layer "F.Cu") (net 3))
 (segment (start 130.797578 86.175) (end 135.312578 81.66) (width 0.1) (layer "F.Cu") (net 3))
 (segment (start 135.312578 81.66) (end 152.62 81.66) (width 0.1) (layer "F.Cu") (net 3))
 (segment (start 152.62 66.42) (end 153.5 65.54) (width 0.1) (layer "F.Cu") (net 3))
 (segment (start 122.94 85.125) (end 130.375 85.125) (width 0.1) (layer "F.Cu") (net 3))
 (segment (start 141.46 74.04) (end 152.62 74.04) (width 0.1) (layer "F.Cu") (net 3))
 (segment (start 122.94 84.075) (end 129.925 84.075) (width 0.1) (layer "F.Cu") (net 3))
 (segment (start 153.5 65.54) (end 156.04 65.54) (width 0.1) (layer "F.Cu") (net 3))
 (segment (start 153.5 73.16) (end 156.04 73.16) (width 0.1) (layer "F.Cu") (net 3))
 (segment (start 147.58 66.42) (end 152.62 66.42) (width 0.1) (layer "F.Cu") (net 3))
 (segment (start 152.62 74.04) (end 153.5 73.16) (width 0.1) (layer "F.Cu") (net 3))
 (segment (start 141 98.5) (end 153.44 98.5) (width 0.1) (layer "F.Cu") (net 24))
 (segment (start 122.94 88.625) (end 131.125 88.625) (width 0.1) (layer "F.Cu") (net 24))
 (segment (start 131.125 88.625) (end 141 98.5) (width 0.1) (layer "F.Cu") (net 24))
 (segment (start 153.44 98.5) (end 153.5 98.56) (width 0.1) (layer "F.Cu") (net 24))
 (segment (start 156.327208 114.4) (end 142.215208 114.4) (width 0.1) (layer "F.Cu") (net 23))
 (segment (start 120.572114 88.275) (end 121.12 88.275) (width 0.1) (layer "F.Cu") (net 23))
 (segment (start 119.755 91.939792) (end 119.755 89.092114) (width 0.1) (layer "F.Cu") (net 23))
 (segment (start 142.215208 114.4) (end 119.755 91.939792) (width 0.1) (layer "F.Cu") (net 23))
 (segment (start 156.04 96.02) (end 158.101 98.081) (width 0.1) (layer "F.Cu") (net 23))
 (segment (start 158.101 98.081) (end 158.101 112.626208) (width 0.1) (layer "F.Cu") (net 23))
 (segment (start 158.101 112.626208) (end 156.327208 114.4) (width 0.1) (layer "F.Cu") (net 23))
 (segment (start 119.755 89.092114) (end 120.572114 88.275) (width 0.1) (layer "F.Cu") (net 23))
 (segment (start 130.675 85.825) (end 137.38 79.12) (width 0.1) (layer "F.Cu") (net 10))
 (segment (start 152.62 79.12) (end 153.5 78.24) (width 0.1) (layer "F.Cu") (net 10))
 (segment (start 122.94 85.825) (end 130.675 85.825) (width 0.1) (layer "F.Cu") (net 10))
 (segment (start 137.38 79.12) (end 152.62 79.12) (width 0.1) (layer "F.Cu") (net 10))
 (segment (start 129.775 83.725) (end 149.62 63.88) (width 0.1) (layer "F.Cu") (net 1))
 (segment (start 122.94 83.725) (end 129.775 83.725) (width 0.1) (layer "F.Cu") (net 1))
 (segment (start 152.62 63.88) (end 153.5 63) (width 0.1) (layer "F.Cu") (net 1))
 (segment (start 149.62 63.88) (end 152.62 63.88) (width 0.1) (layer "F.Cu") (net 1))
 (segment (start 156.971788 57.699) (end 133.523966 57.699) (width 0.1) (layer "F.Cu") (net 16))
 (segment (start 156.04 85.86) (end 159.5 82.4) (width 0.1) (layer "F.Cu") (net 16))
 (segment (start 159.5 82.4) (end 159.5 60.227212) (width 0.1) (layer "F.Cu") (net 16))
 (segment (start 159.5 60.227212) (end 156.971788 57.699) (width 0.1) (layer "F.Cu") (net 16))
 (segment (start 114.995 83.846356) (end 118.023644 86.875) (width 0.1) (layer "F.Cu") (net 16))
 (segment (start 114.995 76.227966) (end 114.995 83.846356) (width 0.1) (layer "F.Cu") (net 16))
 (segment (start 133.523966 57.699) (end 114.995 76.227966) (width 0.1) (layer "F.Cu") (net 16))
 (segment (start 118.023644 86.875) (end 121.12 86.875) (width 0.1) (layer "F.Cu") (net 16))
 (segment (start 122.94 86.875) (end 152.485 86.875) (width 0.1) (layer "F.Cu") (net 15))
 (segment (start 152.485 86.875) (end 153.5 85.86) (width 0.1) (layer "F.Cu") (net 15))
 (segment (start 152.325 87.225) (end 153.5 88.4) (width 0.1) (layer "F.Cu") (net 12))
 (segment (start 154.939 86.961) (end 153.5 88.4) (width 0.1) (layer "F.Cu") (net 12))
 (segment (start 122.94 90.025) (end 130.025 90.025) (width 0.1) (layer "F.Cu") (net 12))
 (segment (start 154.939 81.881) (end 154.939 86.961) (width 0.1) (layer "F.Cu") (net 12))
 (segment (start 152.62 109.6) (end 153.5 108.72) (width 0.1) (layer "F.Cu") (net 12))
 (segment (start 153.5 108.72) (end 156.04 106.18) (width 0.1) (layer "F.Cu") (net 12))
 (segment (start 156.04 80.78) (end 154.939 81.881) (width 0.1) (layer "F.Cu") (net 12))
 (segment (start 122.94 87.225) (end 152.325 87.225) (width 0.1) (layer "F.Cu") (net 12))
 (segment (start 149.6 109.6) (end 152.62 109.6) (width 0.1) (layer "F.Cu") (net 12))
 (segment (start 130.025 90.025) (end 149.6 109.6) (width 0.1) (layer "F.Cu") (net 12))
 (segment (start 143.98 101.98) (end 152.62 101.98) (width 0.1) (layer "F.Cu") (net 26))
 (segment (start 122.94 88.975) (end 130.975 88.975) (width 0.1) (layer "F.Cu") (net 26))
 (segment (start 130.975 88.975) (end 143.98 101.98) (width 0.1) (layer "F.Cu") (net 26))
 (segment (start 152.62 101.98) (end 153.5 101.1) (width 0.1) (layer "F.Cu") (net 26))
 (segment (start 159.001 112.999) (end 156.5 115.5) (width 0.1) (layer "F.Cu") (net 17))
 (segment (start 156.5 115.5) (end 142.041002 115.5) (width 0.1) (layer "F.Cu") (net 17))
 (segment (start 159.001 91.361) (end 159.001 112.999) (width 0.1) (layer "F.Cu") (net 17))
 (segment (start 156.04 88.4) (end 159.001 91.361) (width 0.1) (layer "F.Cu") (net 17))
 (segment (start 118.855 88.717908) (end 120.347908 87.225) (width 0.1) (layer "F.Cu") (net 17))
 (segment (start 120.347908 87.225) (end 121.12 87.225) (width 0.1) (layer "F.Cu") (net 17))
 (segment (start 142.041002 115.5) (end 118.855 92.313998) (width 0.1) (layer "F.Cu") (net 17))
 (segment (start 118.855 92.313998) (end 118.855 88.717908) (width 0.1) (layer "F.Cu") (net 17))
 (segment (start 152.62 104.52) (end 153.5 103.64) (width 0.1) (layer "F.Cu") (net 2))
 (segment (start 122.94 89.325) (end 130.325 89.325) (width 0.1) (layer "F.Cu") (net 2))
 (segment (start 145.52 104.52) (end 152.62 104.52) (width 0.1) (layer "F.Cu") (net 2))
 (segment (start 130.325 89.325) (end 145.52 104.52) (width 0.1) (layer "F.Cu") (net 2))
 (segment (start 156.04 63) (end 154.939 64.101) (width 0.1) (layer "B.Cu") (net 2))
 (segment (start 154.939 64.101) (end 154.939 102.201) (width 0.1) (layer "B.Cu") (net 2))
 (segment (start 154.939 102.201) (end 153.5 103.64) (width 0.1) (layer "B.Cu") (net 2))
 (segment (start 153.42 68) (end 153.5 68.08) (width 0.1) (layer "F.Cu") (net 4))
 (segment (start 122.94 84.425) (end 130.075 84.425) (width 0.1) (layer "F.Cu") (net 4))
 (segment (start 146.5 68) (end 153.42 68) (width 0.1) (layer "F.Cu") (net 4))
 (segment (start 130.075 84.425) (end 146.5 68) (width 0.1) (layer "F.Cu") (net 4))
 (segment (start 131.069084 86.525) (end 134.833084 82.761) (width 0.1) (layer "F.Cu") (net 13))
 (segment (start 152.941 82.761) (end 153.5 83.32) (width 0.1) (layer "F.Cu") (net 13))
 (segment (start 134.833084 82.761) (end 152.941 82.761) (width 0.1) (layer "F.Cu") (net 13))
 (segment (start 122.94 86.525) (end 131.069084 86.525) (width 0.1) (layer "F.Cu") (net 13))
 (segment (start 152.62 112.14) (end 153.5 111.26) (width 0.1) (layer "F.Cu") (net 31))
 (segment (start 129.875 90.375) (end 151.64 112.14) (width 0.1) (layer "F.Cu") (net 31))
 (segment (start 151.64 112.14) (end 152.62 112.14) (width 0.1) (layer "F.Cu") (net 31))
 (segment (start 122.94 90.375) (end 129.875 90.375) (width 0.1) (layer "F.Cu") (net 31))
 (segment (start 139.5 76.5) (end 152.7 76.5) (width 0.1) (layer "F.Cu") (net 8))
 (segment (start 122.94 85.475) (end 130.525 85.475) (width 0.1) (layer "F.Cu") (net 8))
 (segment (start 130.525 85.475) (end 139.5 76.5) (width 0.1) (layer "F.Cu") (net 8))
 (segment (start 152.7 76.5) (end 153.5 75.7) (width 0.1) (layer "F.Cu") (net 8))
 (segment (start 133.773322 58.301) (end 115.597 76.477322) (width 0.1) (layer "F.Cu") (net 11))
 (segment (start 156.04 78.24) (end 158.899 75.381) (width 0.1) (layer "F.Cu") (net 11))
 (segment (start 158.899 60.476154) (end 156.723846 58.301) (width 0.1) (layer "F.Cu") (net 11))
 (segment (start 117.825002 85.825) (end 121.12 85.825) (width 0.1) (layer "F.Cu") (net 11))
 (segment (start 115.597 83.597) (end 117.825002 85.825) (width 0.1) (layer "F.Cu") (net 11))
 (segment (start 115.597 76.477322) (end 115.597 83.597) (width 0.1) (layer "F.Cu") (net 11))
 (segment (start 156.723846 58.301) (end 133.773322 58.301) (width 0.1) (layer "F.Cu") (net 11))
 (segment (start 158.899 75.381) (end 158.899 60.476154) (width 0.1) (layer "F.Cu") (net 11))
 (segment (start 139.959664 96.9) (end 152.62 96.9) (width 0.1) (layer "F.Cu") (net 22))
 (segment (start 122.94 88.275) (end 131.334664 88.275) (width 0.1) (layer "F.Cu") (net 22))
 (segment (start 131.334664 88.275) (end 139.959664 96.9) (width 0.1) (layer "F.Cu") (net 22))
 (segment (start 152.62 96.9) (end 153.5 96.02) (width 0.1) (layer "F.Cu") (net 22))
 (segment (start 156.04 83.32) (end 159.2 80.16) (width 0.1) (layer "F.Cu") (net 14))
 (segment (start 156.848524 58) (end 133.648644 58) (width 0.1) (layer "F.Cu") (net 14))
 (segment (start 118.099324 86.525) (end 121.12 86.525) (width 0.1) (layer "F.Cu") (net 14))
 (segment (start 159.2 60.351476) (end 156.848524 58) (width 0.1) (layer "F.Cu") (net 14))
 (segment (start 115.296 76.352644) (end 115.296 83.721678) (width 0.1) (layer "F.Cu") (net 14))
 (segment (start 133.648644 58) (end 115.296 76.352644) (width 0.1) (layer "F.Cu") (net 14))
 (segment (start 115.296 83.721678) (end 118.099324 86.525) (width 0.1) (layer "F.Cu") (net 14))
 (segment (start 159.2 80.16) (end 159.2 60.351476) (width 0.1) (layer "F.Cu") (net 14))
 (segment (start 122.94 87.925) (end 131.425 87.925) (width 0.1) (layer "F.Cu") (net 20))
 (segment (start 137.86 94.36) (end 152.62 94.36) (width 0.1) (layer "F.Cu") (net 20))
 (segment (start 131.425 87.925) (end 137.86 94.36) (width 0.1) (layer "F.Cu") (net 20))
 (segment (start 152.62 94.36) (end 153.5 93.48) (width 0.1) (layer "F.Cu") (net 20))
 (segment (start 134 59.5) (end 116.5 77) (width 0.1) (layer "F.Cu") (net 5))
 (segment (start 156.04 68.08) (end 157.141 66.979) (width 0.1) (layer "F.Cu") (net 5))
 (segment (start 157.141 66.979) (end 157.141 60.17671) (width 0.1) (layer "F.Cu") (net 5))
 (segment (start 156.46429 59.5) (end 134 59.5) (width 0.1) (layer "F.Cu") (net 5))
 (segment (start 116.5 83.222966) (end 117.702034 84.425) (width 0.1) (layer "F.Cu") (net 5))
 (segment (start 117.702034 84.425) (end 121.12 84.425) (width 0.1) (layer "F.Cu") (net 5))
 (segment (start 157.141 60.17671) (end 156.46429 59.5) (width 0.1) (layer "F.Cu") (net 5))
 (segment (start 116.5 77) (end 116.5 83.222966) (width 0.1) (layer "F.Cu") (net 5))
 (segment (start 158.401 95.841) (end 158.401 112.750472) (width 0.1) (layer "F.Cu") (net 21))
 (segment (start 142.090944 114.7) (end 119.455 92.064056) (width 0.1) (layer "F.Cu") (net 21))
 (segment (start 156.451472 114.7) (end 142.090944 114.7) (width 0.1) (layer "F.Cu") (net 21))
 (segment (start 119.455 88.96785) (end 120.49785 87.925) (width 0.1) (layer "F.Cu") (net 21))
 (segment (start 156.04 93.48) (end 158.401 95.841) (width 0.1) (layer "F.Cu") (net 21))
 (segment (start 120.49785 87.925) (end 121.12 87.925) (width 0.1) (layer "F.Cu") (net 21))
 (segment (start 158.401 112.750472) (end 156.451472 114.7) (width 0.1) (layer "F.Cu") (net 21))
 (segment (start 119.455 92.064056) (end 119.455 88.96785) (width 0.1) (layer "F.Cu") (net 21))
 (segment (start 146.5 106) (end 153.32 106) (width 0.1) (layer "F.Cu") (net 29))
 (segment (start 122.94 89.675) (end 130.175 89.675) (width 0.1) (layer "F.Cu") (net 29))
 (segment (start 153.32 106) (end 153.5 106.18) (width 0.1) (layer "F.Cu") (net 29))
 (segment (start 130.175 89.675) (end 146.5 106) (width 0.1) (layer "F.Cu") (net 29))
 (segment (start 133.801 58.699) (end 115.898 76.602) (width 0.1) (layer "F.Cu") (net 9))
 (segment (start 117.900676 85.475) (end 121.12 85.475) (width 0.1) (layer "F.Cu") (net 9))
 (segment (start 115.898 76.602) (end 115.898 83.472324) (width 0.1) (layer "F.Cu") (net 9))
 (segment (start 158.599 73.141) (end 158.599 60.600418) (width 0.1) (layer "F.Cu") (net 9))
 (segment (start 156.697582 58.699) (end 133.801 58.699) (width 0.1) (layer "F.Cu") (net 9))
 (segment (start 158.599 60.600418) (end 156.697582 58.699) (width 0.1) (layer "F.Cu") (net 9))
 (segment (start 156.04 75.7) (end 158.599 73.141) (width 0.1) (layer "F.Cu") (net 9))
 (segment (start 115.898 83.472324) (end 117.900676 85.475) (width 0.1) (layer "F.Cu") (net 9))
 (segment (start 117.626356 84.775) (end 121.12 84.775) (width 0.1) (layer "F.Cu") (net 7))
 (segment (start 158.299 60.724682) (end 156.574318 59) (width 0.1) (layer "F.Cu") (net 7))
 (segment (start 116.199 83.347644) (end 117.626356 84.775) (width 0.1) (layer "F.Cu") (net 7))
 (segment (start 156.574318 59) (end 134 59) (width 0.1) (layer "F.Cu") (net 7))
 (segment (start 116.199 76.801) (end 116.199 83.347644) (width 0.1) (layer "F.Cu") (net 7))
 (segment (start 158.299 68.361) (end 158.299 60.724682) (width 0.1) (layer "F.Cu") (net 7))
 (segment (start 156.04 70.62) (end 158.299 68.361) (width 0.1) (layer "F.Cu") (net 7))
 (segment (start 134 59) (end 116.199 76.801) (width 0.1) (layer "F.Cu") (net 7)))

